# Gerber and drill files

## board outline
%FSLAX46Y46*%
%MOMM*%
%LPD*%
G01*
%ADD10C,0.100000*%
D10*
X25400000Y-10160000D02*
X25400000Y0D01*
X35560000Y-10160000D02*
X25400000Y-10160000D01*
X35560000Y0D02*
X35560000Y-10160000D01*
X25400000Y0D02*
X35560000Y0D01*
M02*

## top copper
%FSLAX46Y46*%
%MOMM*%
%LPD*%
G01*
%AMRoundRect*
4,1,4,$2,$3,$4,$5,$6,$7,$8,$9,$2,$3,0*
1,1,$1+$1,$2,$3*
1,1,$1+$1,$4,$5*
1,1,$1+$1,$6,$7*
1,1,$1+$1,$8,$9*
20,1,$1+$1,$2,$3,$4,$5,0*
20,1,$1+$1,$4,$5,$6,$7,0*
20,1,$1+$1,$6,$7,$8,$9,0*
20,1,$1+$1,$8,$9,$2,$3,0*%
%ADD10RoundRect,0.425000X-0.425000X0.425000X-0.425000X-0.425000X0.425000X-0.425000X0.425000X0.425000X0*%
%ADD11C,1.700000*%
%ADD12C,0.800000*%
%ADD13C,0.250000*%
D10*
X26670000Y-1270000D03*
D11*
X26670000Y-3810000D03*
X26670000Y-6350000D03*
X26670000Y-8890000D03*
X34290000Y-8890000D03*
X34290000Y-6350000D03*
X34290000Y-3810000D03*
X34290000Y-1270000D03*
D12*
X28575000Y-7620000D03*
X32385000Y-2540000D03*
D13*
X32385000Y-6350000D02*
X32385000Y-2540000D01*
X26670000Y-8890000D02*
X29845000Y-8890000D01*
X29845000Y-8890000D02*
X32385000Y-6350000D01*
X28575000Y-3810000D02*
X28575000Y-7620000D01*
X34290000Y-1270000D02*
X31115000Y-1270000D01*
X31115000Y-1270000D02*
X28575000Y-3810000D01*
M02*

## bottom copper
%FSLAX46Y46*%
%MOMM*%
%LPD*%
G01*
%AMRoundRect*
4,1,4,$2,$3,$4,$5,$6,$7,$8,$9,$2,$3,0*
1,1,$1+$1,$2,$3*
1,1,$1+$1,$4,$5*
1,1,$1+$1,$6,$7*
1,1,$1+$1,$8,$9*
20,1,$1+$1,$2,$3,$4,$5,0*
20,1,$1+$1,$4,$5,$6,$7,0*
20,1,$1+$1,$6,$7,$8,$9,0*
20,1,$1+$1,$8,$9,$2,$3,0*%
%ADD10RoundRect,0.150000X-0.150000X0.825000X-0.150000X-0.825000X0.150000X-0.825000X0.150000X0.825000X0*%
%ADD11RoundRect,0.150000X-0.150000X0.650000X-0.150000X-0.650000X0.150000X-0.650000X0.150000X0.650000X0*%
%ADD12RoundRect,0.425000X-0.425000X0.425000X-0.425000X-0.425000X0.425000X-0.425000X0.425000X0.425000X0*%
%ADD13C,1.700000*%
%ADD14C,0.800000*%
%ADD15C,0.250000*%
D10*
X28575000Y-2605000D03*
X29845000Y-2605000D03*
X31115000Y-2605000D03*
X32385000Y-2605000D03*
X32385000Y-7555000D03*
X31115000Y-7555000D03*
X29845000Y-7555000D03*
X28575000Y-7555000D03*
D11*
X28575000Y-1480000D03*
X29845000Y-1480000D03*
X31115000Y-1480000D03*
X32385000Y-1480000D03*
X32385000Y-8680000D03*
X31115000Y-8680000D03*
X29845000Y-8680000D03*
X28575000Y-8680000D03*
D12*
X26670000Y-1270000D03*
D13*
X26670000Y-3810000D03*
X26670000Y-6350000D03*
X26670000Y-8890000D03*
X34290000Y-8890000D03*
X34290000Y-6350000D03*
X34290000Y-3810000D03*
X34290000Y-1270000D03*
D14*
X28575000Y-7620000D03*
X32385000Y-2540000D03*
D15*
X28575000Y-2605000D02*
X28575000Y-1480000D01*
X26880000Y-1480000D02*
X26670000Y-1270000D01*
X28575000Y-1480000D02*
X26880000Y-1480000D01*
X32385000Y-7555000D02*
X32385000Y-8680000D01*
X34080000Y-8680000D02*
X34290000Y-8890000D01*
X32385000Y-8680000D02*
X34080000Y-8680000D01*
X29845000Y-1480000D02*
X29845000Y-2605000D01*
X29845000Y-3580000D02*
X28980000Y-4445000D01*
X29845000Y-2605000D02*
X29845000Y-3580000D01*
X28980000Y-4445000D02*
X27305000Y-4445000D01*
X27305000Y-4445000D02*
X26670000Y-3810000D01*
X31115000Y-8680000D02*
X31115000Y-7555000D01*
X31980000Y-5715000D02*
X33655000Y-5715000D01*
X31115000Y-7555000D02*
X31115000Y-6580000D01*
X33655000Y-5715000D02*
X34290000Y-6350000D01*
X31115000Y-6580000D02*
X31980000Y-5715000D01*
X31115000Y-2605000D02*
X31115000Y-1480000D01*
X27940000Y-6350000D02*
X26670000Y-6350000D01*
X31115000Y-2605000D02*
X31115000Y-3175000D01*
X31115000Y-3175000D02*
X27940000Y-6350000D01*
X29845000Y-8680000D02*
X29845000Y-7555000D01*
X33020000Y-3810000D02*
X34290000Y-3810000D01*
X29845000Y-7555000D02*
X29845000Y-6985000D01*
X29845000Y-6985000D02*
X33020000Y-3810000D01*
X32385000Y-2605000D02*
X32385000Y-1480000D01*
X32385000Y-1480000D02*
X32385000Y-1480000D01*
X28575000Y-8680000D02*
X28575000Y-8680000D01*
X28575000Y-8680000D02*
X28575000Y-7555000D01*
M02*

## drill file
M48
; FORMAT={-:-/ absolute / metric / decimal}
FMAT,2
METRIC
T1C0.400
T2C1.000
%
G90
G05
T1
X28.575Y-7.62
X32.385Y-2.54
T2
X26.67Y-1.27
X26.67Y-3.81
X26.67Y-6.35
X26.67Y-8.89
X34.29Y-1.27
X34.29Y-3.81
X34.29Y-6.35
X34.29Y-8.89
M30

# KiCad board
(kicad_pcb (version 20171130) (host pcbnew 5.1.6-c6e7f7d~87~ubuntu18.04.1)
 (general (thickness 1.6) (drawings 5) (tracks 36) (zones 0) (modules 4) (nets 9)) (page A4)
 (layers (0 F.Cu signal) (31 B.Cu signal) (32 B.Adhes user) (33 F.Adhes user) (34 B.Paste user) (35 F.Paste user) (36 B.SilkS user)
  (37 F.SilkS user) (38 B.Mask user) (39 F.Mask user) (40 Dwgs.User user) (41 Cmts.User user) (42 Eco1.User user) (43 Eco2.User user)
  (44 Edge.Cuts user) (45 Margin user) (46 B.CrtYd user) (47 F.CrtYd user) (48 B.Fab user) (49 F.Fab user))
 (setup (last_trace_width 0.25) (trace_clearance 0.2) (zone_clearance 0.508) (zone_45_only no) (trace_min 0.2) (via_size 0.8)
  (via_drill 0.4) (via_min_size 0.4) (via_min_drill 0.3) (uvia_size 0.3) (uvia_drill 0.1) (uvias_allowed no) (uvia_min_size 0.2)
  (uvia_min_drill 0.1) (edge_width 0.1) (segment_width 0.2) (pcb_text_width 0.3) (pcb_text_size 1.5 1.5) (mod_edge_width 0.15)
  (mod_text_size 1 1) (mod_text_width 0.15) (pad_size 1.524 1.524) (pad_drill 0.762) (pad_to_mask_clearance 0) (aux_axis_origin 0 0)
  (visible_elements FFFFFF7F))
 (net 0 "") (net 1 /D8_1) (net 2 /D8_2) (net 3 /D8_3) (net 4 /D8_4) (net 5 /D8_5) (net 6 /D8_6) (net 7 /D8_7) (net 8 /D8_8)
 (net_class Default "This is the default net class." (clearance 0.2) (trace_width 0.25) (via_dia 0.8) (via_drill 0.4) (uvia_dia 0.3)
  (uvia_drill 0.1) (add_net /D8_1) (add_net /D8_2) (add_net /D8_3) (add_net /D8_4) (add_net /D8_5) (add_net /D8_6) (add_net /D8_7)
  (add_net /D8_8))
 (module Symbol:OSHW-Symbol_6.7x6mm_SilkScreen (layer F.Cu) (at 30.48 4.826)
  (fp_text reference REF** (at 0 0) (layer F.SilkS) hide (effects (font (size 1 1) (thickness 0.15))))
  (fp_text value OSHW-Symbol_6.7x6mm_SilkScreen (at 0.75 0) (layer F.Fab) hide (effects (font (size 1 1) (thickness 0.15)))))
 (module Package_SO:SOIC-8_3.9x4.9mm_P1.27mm (layer B.Cu) (at 30.48 5.08 270)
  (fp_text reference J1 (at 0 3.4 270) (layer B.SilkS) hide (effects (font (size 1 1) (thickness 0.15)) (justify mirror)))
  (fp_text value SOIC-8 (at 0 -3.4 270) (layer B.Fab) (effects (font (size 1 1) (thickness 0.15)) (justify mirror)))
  (pad 1 smd roundrect (at -2.475 1.905 270) (size 1.95 0.6) (layers B.Cu B.Paste B.Mask) (roundrect_rratio 0.25) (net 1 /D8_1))
  (pad 2 smd roundrect (at -2.475 0.635 270) (size 1.95 0.6) (layers B.Cu B.Paste B.Mask) (roundrect_rratio 0.25) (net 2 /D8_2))
  (pad 3 smd roundrect (at -2.475 -0.635 270) (size 1.95 0.6) (layers B.Cu B.Paste B.Mask) (roundrect_rratio 0.25) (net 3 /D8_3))
  (pad 4 smd roundrect (at -2.475 -1.905 270) (size 1.95 0.6) (layers B.Cu B.Paste B.Mask) (roundrect_rratio 0.25) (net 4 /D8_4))
  (pad 5 smd roundrect (at 2.475 -1.905 270) (size 1.95 0.6) (layers B.Cu B.Paste B.Mask) (roundrect_rratio 0.25) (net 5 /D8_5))
  (pad 6 smd roundrect (at 2.475 -0.635 270) (size 1.95 0.6) (layers B.Cu B.Paste B.Mask) (roundrect_rratio 0.25) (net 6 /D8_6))
  (pad 7 smd roundrect (at 2.475 0.635 270) (size 1.95 0.6) (layers B.Cu B.Paste B.Mask) (roundrect_rratio 0.25) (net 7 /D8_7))
  (pad 8 smd roundrect (at 2.475 1.905 270) (size 1.95 0.6) (layers B.Cu B.Paste B.Mask) (roundrect_rratio 0.25) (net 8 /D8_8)))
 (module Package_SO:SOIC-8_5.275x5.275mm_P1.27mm (layer B.Cu) (at 30.48 5.08 270)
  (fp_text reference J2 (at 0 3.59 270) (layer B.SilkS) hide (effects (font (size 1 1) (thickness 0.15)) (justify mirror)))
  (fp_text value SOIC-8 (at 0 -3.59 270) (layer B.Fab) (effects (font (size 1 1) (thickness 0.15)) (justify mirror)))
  (pad 1 smd roundrect (at -3.6 1.905 270) (size 1.6 0.6) (layers B.Cu B.Paste B.Mask) (roundrect_rratio 0.25) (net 1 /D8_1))
  (pad 2 smd roundrect (at -3.6 0.635 270) (size 1.6 0.6) (layers B.Cu B.Paste B.Mask) (roundrect_rratio 0.25) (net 2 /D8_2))
  (pad 3 smd roundrect (at -3.6 -0.635 270) (size 1.6 0.6) (layers B.Cu B.Paste B.Mask) (roundrect_rratio 0.25) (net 3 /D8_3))
  (pad 4 smd roundrect (at -3.6 -1.905 270) (size 1.6 0.6) (layers B.Cu B.Paste B.Mask) (roundrect_rratio 0.25) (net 4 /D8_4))
  (pad 5 smd roundrect (at 3.6 -1.905 270) (size 1.6 0.6) (layers B.Cu B.Paste B.Mask) (roundrect_rratio 0.25) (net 5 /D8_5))
  (pad 6 smd roundrect (at 3.6 -0.635 270) (size 1.6 0.6) (layers B.Cu B.Paste B.Mask) (roundrect_rratio 0.25) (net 6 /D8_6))
  (pad 7 smd roundrect (at 3.6 0.635 270) (size 1.6 0.6) (layers B.Cu B.Paste B.Mask) (roundrect_rratio 0.25) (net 7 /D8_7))
  (pad 8 smd roundrect (at 3.6 1.905 270) (size 1.6 0.6) (layers B.Cu B.Paste B.Mask) (roundrect_rratio 0.25) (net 8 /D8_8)))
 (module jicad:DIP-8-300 (layer F.Cu) (at 26.67 1.27 270)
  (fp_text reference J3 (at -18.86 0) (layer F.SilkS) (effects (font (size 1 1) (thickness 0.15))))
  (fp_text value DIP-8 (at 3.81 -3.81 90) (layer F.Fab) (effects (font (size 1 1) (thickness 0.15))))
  (pad 1 thru_hole roundrect (at 0 0 270) (size 1.7 1.7) (drill 1) (layers *.Cu *.Mask) (roundrect_rratio 0.25) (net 1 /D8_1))
  (pad 2 thru_hole circle (at 2.54 0 270) (size 1.7 1.7) (drill 1) (layers *.Cu *.Mask) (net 2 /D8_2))
  (pad 3 thru_hole circle (at 5.08 0 270) (size 1.7 1.7) (drill 1) (layers *.Cu *.Mask) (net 3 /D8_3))
  (pad 4 thru_hole circle (at 7.62 0 270) (size 1.7 1.7) (drill 1) (layers *.Cu *.Mask) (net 4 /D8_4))
  (pad 5 thru_hole circle (at 7.62 -7.62 90) (size 1.7 1.7) (drill 1) (layers *.Cu *.Mask) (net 5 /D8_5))
  (pad 6 thru_hole circle (at 5.08 -7.62 90) (size 1.7 1.7) (drill 1) (layers *.Cu *.Mask) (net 6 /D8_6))
  (pad 7 thru_hole circle (at 2.54 -7.62 90) (size 1.7 1.7) (drill 1) (layers *.Cu *.Mask) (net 7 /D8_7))
  (pad 8 thru_hole circle (at 0 -7.62 90) (size 1.7 1.7) (drill 1) (layers *.Cu *.Mask) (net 8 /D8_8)))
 (gr_line (start 25.4 10.16) (end 25.4 0) (layer Edge.Cuts) (width 0.1))
 (gr_line (start 35.56 10.16) (end 25.4 10.16) (layer Edge.Cuts) (width 0.1))
 (gr_line (start 35.56 0) (end 35.56 10.16) (layer Edge.Cuts) (width 0.1))
 (gr_line (start 25.4 0) (end 35.56 0) (layer Edge.Cuts) (width 0.1))
 (via (at 28.575 7.62) (size 0.8) (drill 0.4) (layers F.Cu B.Cu) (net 8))
 (via (at 32.385 2.54) (size 0.8) (drill 0.4) (layers F.Cu B.Cu) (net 4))
 (segment (start 28.575 2.605) (end 28.575 1.48) (width 0.25) (layer B.Cu) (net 1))
 (segment (start 26.88 1.48) (end 26.67 1.27) (width 0.25) (layer B.Cu) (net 1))
 (segment (start 28.575 1.48) (end 26.88 1.48) (width 0.25) (layer B.Cu) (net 1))
 (segment (start 32.385 7.555) (end 32.385 8.68) (width 0.25) (layer B.Cu) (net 5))
 (segment (start 34.08 8.68) (end 34.29 8.89) (width 0.25) (layer B.Cu) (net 5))
 (segment (start 32.385 8.68) (end 34.08 8.68) (width 0.25) (layer B.Cu) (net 5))
 (segment (start 29.845 1.48) (end 29.845 2.605) (width 0.25) (layer B.Cu) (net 2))
 (segment (start 29.845 3.58) (end 28.98 4.445) (width 0.25) (layer B.Cu) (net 2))
 (segment (start 29.845 2.605) (end 29.845 3.58) (width 0.25) (layer B.Cu) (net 2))
 (segment (start 28.98 4.445) (end 27.305 4.445) (width 0.25) (layer B.Cu) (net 2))
 (segment (start 27.305 4.445) (end 26.67 3.81) (width 0.25) (layer B.Cu) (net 2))
 (segment (start 31.115 8.68) (end 31.115 7.555) (width 0.25) (layer B.Cu) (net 6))
 (segment (start 31.98 5.715) (end 33.655 5.715) (width 0.25) (layer B.Cu) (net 6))
 (segment (start 31.115 7.555) (end 31.115 6.58) (width 0.25) (layer B.Cu) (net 6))
 (segment (start 33.655 5.715) (end 34.29 6.35) (width 0.25) (layer B.Cu) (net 6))
 (segment (start 31.115 6.58) (end 31.98 5.715) (width 0.25) (layer B.Cu) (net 6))
 (segment (start 31.115 2.605) (end 31.115 1.48) (width 0.25) (layer B.Cu) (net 3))
 (segment (start 27.94 6.35) (end 26.67 6.35) (width 0.25) (layer B.Cu) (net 3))
 (segment (start 31.115 2.605) (end 31.115 3.175) (width 0.25) (layer B.Cu) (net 3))
 (segment (start 31.115 3.175) (end 27.94 6.35) (width 0.25) (layer B.Cu) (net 3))
 (segment (start 29.845 8.68) (end 29.845 7.555) (width 0.25) (layer B.Cu) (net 7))
 (segment (start 33.02 3.81) (end 34.29 3.81) (width 0.25) (layer B.Cu) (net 7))
 (segment (start 29.845 7.555) (end 29.845 6.985) (width 0.25) (layer B.Cu) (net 7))
 (segment (start 29.845 6.985) (end 33.02 3.81) (width 0.25) (layer B.Cu) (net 7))
 (segment (start 32.385 2.605) (end 32.385 1.48) (width 0.25) (layer B.Cu) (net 4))
 (segment (start 32.385 1.48) (end 32.385 1.48) (width 0.25) (layer B.Cu) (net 4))
 (segment (start 32.385 6.35) (end 32.385 2.54) (width 0.25) (layer F.Cu) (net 4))
 (segment (start 26.67 8.89) (end 29.845 8.89) (width 0.25) (layer F.Cu) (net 4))
 (segment (start 29.845 8.89) (end 32.385 6.35) (width 0.25) (layer F.Cu) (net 4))
 (segment (start 28.575 8.68) (end 28.575 8.68) (width 0.25) (layer B.Cu) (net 8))
 (segment (start 28.575 8.68) (end 28.575 7.555) (width 0.25) (layer B.Cu) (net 8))
 (segment (start 28.575 3.81) (end 28.575 7.62) (width 0.25) (layer F.Cu) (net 8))
 (segment (start 34.29 1.27) (end 31.115 1.27) (width 0.25) (layer F.Cu) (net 8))
 (segment (start 31.115 1.27) (end 28.575 3.81) (width 0.25) (layer F.Cu) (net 8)))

